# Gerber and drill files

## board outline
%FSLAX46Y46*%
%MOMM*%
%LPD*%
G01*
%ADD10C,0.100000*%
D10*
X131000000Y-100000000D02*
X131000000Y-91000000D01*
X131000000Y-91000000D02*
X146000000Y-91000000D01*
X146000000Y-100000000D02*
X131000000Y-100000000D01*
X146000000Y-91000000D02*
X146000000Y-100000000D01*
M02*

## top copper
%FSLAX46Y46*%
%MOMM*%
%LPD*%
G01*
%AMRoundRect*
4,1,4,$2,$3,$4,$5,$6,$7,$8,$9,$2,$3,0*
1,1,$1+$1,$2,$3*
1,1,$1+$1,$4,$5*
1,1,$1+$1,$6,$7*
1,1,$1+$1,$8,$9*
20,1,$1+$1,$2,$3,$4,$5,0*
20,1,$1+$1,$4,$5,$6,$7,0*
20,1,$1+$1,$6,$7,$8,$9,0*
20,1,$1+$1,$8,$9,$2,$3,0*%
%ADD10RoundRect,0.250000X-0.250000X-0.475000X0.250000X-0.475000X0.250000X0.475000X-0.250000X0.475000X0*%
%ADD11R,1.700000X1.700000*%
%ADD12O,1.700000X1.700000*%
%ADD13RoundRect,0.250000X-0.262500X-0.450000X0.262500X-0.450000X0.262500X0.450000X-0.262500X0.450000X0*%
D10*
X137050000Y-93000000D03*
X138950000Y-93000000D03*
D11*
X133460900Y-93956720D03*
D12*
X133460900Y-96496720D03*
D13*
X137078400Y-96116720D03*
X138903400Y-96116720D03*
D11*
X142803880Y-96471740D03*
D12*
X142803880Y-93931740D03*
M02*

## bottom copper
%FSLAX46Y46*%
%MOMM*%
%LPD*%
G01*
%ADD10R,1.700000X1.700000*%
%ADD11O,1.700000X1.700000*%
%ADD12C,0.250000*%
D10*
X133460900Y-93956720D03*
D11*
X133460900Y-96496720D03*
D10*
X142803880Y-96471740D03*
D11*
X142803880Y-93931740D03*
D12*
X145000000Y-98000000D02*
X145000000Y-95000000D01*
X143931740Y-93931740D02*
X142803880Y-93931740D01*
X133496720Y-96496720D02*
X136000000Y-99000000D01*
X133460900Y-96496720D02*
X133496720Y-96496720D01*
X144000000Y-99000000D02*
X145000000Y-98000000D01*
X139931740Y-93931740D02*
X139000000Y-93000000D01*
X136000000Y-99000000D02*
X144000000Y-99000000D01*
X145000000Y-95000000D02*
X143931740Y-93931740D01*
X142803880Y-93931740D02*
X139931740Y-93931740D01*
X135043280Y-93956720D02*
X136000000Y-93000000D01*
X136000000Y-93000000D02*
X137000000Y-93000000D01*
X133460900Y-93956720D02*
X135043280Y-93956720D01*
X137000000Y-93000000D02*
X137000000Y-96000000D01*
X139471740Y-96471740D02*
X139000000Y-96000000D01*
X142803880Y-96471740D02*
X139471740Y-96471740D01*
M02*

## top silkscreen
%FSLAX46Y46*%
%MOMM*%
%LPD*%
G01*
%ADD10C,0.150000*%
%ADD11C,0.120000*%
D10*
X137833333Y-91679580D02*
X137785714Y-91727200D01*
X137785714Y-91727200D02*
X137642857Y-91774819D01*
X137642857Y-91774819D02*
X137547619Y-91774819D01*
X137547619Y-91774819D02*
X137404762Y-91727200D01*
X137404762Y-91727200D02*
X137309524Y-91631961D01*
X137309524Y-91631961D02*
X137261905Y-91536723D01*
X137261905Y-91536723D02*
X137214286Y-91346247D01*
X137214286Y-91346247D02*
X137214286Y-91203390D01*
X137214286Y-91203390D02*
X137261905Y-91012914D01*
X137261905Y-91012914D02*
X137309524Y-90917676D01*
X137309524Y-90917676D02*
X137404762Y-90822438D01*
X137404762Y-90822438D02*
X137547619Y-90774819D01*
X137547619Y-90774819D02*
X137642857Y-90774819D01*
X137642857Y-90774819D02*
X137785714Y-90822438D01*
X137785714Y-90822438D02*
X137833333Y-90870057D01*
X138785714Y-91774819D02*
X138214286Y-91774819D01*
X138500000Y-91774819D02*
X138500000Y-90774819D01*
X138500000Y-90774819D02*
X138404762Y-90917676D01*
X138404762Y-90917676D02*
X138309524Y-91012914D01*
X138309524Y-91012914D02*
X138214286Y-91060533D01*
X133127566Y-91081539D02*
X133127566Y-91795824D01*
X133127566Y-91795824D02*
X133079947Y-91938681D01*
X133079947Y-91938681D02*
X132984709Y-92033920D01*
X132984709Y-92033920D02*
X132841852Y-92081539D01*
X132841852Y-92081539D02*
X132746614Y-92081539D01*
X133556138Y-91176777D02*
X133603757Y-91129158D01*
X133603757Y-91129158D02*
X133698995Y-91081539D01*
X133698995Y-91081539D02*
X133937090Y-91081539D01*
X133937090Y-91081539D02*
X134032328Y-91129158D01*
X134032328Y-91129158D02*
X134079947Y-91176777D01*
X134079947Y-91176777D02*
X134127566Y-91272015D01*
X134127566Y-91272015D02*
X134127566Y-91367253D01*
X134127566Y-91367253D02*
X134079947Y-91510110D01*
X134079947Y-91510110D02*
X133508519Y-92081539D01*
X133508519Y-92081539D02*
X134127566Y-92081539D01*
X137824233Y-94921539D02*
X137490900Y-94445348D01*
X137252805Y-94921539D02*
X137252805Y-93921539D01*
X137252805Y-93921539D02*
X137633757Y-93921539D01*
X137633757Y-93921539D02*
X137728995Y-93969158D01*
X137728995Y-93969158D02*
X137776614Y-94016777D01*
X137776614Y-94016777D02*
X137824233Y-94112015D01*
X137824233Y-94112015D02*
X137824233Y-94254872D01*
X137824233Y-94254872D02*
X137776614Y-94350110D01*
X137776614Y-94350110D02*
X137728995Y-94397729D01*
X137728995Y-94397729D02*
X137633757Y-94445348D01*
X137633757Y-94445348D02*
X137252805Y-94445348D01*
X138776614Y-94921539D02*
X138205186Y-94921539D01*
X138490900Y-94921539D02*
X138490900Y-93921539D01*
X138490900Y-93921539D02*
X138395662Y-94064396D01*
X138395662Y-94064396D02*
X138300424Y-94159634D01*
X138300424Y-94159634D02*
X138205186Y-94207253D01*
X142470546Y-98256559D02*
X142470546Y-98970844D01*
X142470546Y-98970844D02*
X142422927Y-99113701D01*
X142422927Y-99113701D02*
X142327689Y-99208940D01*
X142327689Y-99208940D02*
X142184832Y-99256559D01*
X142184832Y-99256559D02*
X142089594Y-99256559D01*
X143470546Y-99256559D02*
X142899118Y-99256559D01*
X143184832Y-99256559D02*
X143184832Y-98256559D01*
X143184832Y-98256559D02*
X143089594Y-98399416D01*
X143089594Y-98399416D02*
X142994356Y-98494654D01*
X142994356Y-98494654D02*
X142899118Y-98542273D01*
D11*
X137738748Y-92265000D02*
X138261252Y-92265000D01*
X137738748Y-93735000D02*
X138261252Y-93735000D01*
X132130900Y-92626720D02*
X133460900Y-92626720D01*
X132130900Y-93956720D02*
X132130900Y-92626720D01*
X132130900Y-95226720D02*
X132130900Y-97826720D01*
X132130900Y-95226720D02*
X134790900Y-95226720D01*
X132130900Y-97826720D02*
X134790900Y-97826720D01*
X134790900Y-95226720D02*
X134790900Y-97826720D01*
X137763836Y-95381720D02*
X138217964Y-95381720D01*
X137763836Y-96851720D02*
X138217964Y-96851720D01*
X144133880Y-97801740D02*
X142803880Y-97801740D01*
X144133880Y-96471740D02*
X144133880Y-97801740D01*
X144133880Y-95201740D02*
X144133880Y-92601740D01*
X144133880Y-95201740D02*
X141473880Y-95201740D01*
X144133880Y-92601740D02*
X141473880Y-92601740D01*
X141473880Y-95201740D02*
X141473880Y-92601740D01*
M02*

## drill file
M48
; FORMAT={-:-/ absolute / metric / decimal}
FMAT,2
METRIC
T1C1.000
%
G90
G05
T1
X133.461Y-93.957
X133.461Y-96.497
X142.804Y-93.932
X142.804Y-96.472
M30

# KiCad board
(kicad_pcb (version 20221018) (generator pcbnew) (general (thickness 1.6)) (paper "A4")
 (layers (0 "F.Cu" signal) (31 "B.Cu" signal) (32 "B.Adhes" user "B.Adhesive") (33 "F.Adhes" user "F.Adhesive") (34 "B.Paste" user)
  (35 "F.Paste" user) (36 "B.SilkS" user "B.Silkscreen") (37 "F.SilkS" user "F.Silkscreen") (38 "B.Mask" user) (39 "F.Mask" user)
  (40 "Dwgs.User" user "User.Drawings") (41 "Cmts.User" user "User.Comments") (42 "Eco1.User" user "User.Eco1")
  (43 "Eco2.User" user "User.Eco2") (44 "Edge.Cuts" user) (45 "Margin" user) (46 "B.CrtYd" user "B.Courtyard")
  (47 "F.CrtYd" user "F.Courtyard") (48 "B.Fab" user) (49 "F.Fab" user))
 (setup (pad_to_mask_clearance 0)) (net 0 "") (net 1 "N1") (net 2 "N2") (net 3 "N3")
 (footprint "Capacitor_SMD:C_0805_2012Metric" (layer "F.Cu") (at 138 93)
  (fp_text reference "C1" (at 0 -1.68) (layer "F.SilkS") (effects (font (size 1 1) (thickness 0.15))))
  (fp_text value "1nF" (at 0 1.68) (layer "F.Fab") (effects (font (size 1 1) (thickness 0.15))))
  (fp_line (start -0.261252 -0.735) (end 0.261252 -0.735) (stroke (width 0.12) (type solid)) (layer "F.SilkS"))
  (fp_line (start -0.261252 0.735) (end 0.261252 0.735) (stroke (width 0.12) (type solid)) (layer "F.SilkS"))
  (pad "1" smd roundrect (at -0.95 0) (size 1 1.45) (layers "F.Cu" "F.Paste" "F.Mask") (roundrect_rratio 0.25) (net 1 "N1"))
  (pad "2" smd roundrect (at 0.95 0) (size 1 1.45) (layers "F.Cu" "F.Paste" "F.Mask") (roundrect_rratio 0.25) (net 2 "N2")))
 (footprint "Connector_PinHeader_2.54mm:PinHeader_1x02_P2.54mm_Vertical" (layer "F.Cu") (at 133.4609 93.95672)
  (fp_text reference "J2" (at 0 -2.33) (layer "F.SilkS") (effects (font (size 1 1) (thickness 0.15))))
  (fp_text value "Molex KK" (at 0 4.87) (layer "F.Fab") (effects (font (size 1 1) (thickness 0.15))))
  (fp_line (start -1.33 -1.33) (end 0 -1.33) (stroke (width 0.12) (type solid)) (layer "F.SilkS"))
  (fp_line (start -1.33 0) (end -1.33 -1.33) (stroke (width 0.12) (type solid)) (layer "F.SilkS"))
  (fp_line (start -1.33 1.27) (end -1.33 3.87) (stroke (width 0.12) (type solid)) (layer "F.SilkS"))
  (fp_line (start -1.33 1.27) (end 1.33 1.27) (stroke (width 0.12) (type solid)) (layer "F.SilkS"))
  (fp_line (start -1.33 3.87) (end 1.33 3.87) (stroke (width 0.12) (type solid)) (layer "F.SilkS"))
  (fp_line (start 1.33 1.27) (end 1.33 3.87) (stroke (width 0.12) (type solid)) (layer "F.SilkS"))
  (pad "1" thru_hole rect (at 0 0) (size 1.7 1.7) (drill 1) (layers "*.Cu" "*.Mask") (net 1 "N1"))
  (pad "2" thru_hole oval (at 0 2.54) (size 1.7 1.7) (drill 1) (layers "*.Cu" "*.Mask") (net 2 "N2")))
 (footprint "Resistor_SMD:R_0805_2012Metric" (layer "F.Cu") (at 137.9909 96.11672)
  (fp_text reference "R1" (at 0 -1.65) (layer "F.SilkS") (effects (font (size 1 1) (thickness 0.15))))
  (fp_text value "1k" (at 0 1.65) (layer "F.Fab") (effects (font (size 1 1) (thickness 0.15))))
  (fp_line (start -0.227064 -0.735) (end 0.227064 -0.735) (stroke (width 0.12) (type solid)) (layer "F.SilkS"))
  (fp_line (start -0.227064 0.735) (end 0.227064 0.735) (stroke (width 0.12) (type solid)) (layer "F.SilkS"))
  (pad "1" smd roundrect (at -0.9125 0) (size 1.025 1.4) (layers "F.Cu" "F.Paste" "F.Mask") (roundrect_rratio 0.243902) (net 1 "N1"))
  (pad "2" smd roundrect (at 0.9125 0) (size 1.025 1.4) (layers "F.Cu" "F.Paste" "F.Mask") (roundrect_rratio 0.243902) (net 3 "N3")))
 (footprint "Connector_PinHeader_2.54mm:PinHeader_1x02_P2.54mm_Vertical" (layer "F.Cu") (at 142.80388 96.47174 180)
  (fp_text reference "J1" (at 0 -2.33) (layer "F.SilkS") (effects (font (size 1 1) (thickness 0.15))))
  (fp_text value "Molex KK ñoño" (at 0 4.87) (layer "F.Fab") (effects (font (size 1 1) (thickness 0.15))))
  (fp_line (start -1.33 -1.33) (end 0 -1.33) (stroke (width 0.12) (type solid)) (layer "F.SilkS"))
  (fp_line (start -1.33 0) (end -1.33 -1.33) (stroke (width 0.12) (type solid)) (layer "F.SilkS"))
  (fp_line (start -1.33 1.27) (end -1.33 3.87) (stroke (width 0.12) (type solid)) (layer "F.SilkS"))
  (fp_line (start -1.33 1.27) (end 1.33 1.27) (stroke (width 0.12) (type solid)) (layer "F.SilkS"))
  (fp_line (start -1.33 3.87) (end 1.33 3.87) (stroke (width 0.12) (type solid)) (layer "F.SilkS"))
  (fp_line (start 1.33 1.27) (end 1.33 3.87) (stroke (width 0.12) (type solid)) (layer "F.SilkS"))
  (pad "1" thru_hole rect (at 0 0 180) (size 1.7 1.7) (drill 1) (layers "*.Cu" "*.Mask") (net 3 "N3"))
  (pad "2" thru_hole oval (at 0 2.54 180) (size 1.7 1.7) (drill 1) (layers "*.Cu" "*.Mask") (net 2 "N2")))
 (gr_line (start 131 100) (end 131 91) (stroke (width 0.1) (type solid)) (layer "Edge.Cuts"))
 (gr_line (start 131 91) (end 146 91) (stroke (width 0.1) (type solid)) (layer "Edge.Cuts"))
 (gr_line (start 146 100) (end 131 100) (stroke (width 0.1) (type solid)) (layer "Edge.Cuts"))
 (gr_line (start 146 91) (end 146 100) (stroke (width 0.1) (type solid)) (layer "Edge.Cuts"))
 (segment (start 145 98) (end 145 95) (width 0.25) (layer "B.Cu") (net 2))
 (segment (start 143.93174 93.93174) (end 142.80388 93.93174) (width 0.25) (layer "B.Cu") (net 2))
 (segment (start 133.49672 96.49672) (end 136 99) (width 0.25) (layer "B.Cu") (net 2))
 (segment (start 133.4609 96.49672) (end 133.49672 96.49672) (width 0.25) (layer "B.Cu") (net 2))
 (segment (start 144 99) (end 145 98) (width 0.25) (layer "B.Cu") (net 2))
 (segment (start 139.93174 93.93174) (end 139 93) (width 0.25) (layer "B.Cu") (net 2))
 (segment (start 136 99) (end 144 99) (width 0.25) (layer "B.Cu") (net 2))
 (segment (start 145 95) (end 143.93174 93.93174) (width 0.25) (layer "B.Cu") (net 2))
 (segment (start 142.80388 93.93174) (end 139.93174 93.93174) (width 0.25) (layer "B.Cu") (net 2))
 (segment (start 135.04328 93.95672) (end 136 93) (width 0.25) (layer "B.Cu") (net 1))
 (segment (start 136 93) (end 137 93) (width 0.25) (layer "B.Cu") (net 1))
 (segment (start 133.4609 93.95672) (end 135.04328 93.95672) (width 0.25) (layer "B.Cu") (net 1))
 (segment (start 137 93) (end 137 96) (width 0.25) (layer "B.Cu") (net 1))
 (segment (start 139.47174 96.47174) (end 139 96) (width 0.25) (layer "B.Cu") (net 3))
 (segment (start 142.80388 96.47174) (end 139.47174 96.47174) (width 0.25) (layer "B.Cu") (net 3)))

